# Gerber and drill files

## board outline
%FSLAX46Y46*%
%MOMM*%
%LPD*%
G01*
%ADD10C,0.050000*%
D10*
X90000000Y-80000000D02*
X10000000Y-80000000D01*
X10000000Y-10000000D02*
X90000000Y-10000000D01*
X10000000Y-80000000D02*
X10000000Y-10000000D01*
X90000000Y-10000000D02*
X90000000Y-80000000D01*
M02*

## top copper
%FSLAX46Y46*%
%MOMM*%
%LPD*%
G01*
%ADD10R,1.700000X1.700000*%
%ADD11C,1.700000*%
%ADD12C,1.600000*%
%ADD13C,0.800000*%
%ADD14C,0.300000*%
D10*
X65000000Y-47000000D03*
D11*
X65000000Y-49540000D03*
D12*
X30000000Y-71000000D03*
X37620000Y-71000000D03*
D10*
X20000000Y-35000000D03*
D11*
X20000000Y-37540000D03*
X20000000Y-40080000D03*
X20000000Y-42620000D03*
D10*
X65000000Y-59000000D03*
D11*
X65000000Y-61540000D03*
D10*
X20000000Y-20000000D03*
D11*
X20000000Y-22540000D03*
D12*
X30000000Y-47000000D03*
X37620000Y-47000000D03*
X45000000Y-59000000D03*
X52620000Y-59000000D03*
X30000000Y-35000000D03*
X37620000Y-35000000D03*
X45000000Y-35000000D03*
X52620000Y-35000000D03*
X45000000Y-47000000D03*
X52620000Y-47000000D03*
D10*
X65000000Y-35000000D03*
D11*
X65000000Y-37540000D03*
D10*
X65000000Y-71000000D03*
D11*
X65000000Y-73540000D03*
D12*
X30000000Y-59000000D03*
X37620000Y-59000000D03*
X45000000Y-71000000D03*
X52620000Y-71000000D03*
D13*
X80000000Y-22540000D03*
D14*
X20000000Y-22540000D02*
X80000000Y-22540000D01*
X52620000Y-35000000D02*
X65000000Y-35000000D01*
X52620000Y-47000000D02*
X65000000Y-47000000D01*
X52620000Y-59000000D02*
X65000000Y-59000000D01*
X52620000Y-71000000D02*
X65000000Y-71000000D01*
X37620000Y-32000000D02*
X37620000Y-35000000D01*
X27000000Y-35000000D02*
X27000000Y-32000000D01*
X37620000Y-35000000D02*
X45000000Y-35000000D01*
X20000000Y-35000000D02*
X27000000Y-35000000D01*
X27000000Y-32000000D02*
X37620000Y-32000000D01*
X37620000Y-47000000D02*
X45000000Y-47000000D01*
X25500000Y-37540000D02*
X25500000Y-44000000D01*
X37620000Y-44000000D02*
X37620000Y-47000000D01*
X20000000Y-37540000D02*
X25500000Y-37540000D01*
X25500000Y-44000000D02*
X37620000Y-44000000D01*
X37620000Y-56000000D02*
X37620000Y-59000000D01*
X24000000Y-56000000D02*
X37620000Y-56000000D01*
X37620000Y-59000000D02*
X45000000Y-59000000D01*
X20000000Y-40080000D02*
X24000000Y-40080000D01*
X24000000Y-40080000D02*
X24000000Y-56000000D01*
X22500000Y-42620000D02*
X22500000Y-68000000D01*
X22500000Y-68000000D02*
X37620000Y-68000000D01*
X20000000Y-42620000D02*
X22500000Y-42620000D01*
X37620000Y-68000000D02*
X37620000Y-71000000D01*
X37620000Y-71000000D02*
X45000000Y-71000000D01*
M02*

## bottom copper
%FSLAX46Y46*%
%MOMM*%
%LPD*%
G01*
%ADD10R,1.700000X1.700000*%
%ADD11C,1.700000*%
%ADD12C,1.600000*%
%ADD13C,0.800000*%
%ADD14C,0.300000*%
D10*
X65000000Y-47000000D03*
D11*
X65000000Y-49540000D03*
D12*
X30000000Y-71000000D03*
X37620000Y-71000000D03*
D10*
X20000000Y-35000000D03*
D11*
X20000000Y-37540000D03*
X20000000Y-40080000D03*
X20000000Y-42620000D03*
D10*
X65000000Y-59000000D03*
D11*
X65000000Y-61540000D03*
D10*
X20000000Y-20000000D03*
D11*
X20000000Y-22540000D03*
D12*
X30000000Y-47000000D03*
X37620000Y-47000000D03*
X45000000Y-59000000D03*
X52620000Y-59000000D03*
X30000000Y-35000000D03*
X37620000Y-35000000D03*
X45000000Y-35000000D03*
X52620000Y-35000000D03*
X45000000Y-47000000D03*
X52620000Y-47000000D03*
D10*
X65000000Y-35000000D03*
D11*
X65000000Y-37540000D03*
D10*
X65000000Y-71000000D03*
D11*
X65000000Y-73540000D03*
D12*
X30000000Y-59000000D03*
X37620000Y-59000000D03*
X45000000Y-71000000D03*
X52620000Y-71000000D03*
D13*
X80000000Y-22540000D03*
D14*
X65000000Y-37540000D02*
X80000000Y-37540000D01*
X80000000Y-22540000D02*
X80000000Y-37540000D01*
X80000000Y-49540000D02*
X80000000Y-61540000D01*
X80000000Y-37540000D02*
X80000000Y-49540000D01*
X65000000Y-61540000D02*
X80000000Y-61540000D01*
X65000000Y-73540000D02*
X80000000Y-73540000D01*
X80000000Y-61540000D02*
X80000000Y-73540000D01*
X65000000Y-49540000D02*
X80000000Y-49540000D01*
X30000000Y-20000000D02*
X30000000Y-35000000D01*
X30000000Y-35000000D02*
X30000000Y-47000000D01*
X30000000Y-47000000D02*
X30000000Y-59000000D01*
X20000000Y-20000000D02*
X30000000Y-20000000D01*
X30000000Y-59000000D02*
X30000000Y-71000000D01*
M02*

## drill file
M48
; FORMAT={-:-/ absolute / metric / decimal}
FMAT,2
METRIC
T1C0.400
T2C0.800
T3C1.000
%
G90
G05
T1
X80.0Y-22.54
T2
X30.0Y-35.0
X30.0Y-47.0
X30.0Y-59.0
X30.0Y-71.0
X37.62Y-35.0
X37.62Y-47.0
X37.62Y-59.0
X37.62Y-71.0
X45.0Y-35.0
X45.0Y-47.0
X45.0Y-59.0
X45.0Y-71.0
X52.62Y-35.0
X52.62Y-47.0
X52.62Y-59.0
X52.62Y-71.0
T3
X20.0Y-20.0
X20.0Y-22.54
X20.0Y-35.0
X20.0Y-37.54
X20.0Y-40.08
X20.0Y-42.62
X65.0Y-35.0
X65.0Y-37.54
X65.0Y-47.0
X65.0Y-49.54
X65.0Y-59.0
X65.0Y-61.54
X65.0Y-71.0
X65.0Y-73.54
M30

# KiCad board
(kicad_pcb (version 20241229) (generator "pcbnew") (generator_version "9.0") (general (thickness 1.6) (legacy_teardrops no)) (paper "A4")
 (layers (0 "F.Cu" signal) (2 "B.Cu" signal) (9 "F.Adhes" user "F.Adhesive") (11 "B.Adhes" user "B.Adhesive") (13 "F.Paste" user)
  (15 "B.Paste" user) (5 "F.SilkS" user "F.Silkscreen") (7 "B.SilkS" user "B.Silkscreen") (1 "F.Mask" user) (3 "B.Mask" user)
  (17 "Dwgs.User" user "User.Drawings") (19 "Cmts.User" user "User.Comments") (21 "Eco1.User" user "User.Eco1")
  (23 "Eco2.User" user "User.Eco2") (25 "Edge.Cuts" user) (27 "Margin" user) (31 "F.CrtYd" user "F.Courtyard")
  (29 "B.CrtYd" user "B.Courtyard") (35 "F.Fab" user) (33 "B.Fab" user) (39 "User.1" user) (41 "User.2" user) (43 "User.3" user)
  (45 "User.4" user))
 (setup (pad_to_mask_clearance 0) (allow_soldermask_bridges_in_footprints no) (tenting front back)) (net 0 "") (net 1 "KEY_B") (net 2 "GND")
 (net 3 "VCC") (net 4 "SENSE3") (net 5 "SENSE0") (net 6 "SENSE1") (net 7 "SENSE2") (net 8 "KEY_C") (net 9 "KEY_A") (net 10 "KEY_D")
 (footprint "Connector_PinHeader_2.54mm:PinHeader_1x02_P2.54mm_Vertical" (layer "F.Cu") (at 65 47)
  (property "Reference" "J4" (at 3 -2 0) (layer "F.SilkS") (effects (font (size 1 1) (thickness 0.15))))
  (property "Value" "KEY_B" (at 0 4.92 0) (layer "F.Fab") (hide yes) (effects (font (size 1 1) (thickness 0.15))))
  (pad "1" thru_hole rect (at 0 0) (size 1.7 1.7) (drill 1) (layers "*.Cu" "*.Mask") (remove_unused_layers no) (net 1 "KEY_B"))
  (pad "2" thru_hole circle (at 0 2.54) (size 1.7 1.7) (drill 1) (layers "*.Cu" "*.Mask") (remove_unused_layers no) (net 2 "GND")))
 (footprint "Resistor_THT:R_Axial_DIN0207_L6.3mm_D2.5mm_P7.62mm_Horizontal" (layer "F.Cu") (at 30 71)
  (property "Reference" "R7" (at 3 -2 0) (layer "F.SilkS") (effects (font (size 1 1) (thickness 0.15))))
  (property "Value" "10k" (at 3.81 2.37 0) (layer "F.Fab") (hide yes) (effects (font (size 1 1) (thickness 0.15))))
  (pad "1" thru_hole circle (at 0 0) (size 1.6 1.6) (drill 0.8) (layers "*.Cu" "*.Mask") (remove_unused_layers no) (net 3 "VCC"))
  (pad "2" thru_hole circle (at 7.62 0) (size 1.6 1.6) (drill 0.8) (layers "*.Cu" "*.Mask") (remove_unused_layers no) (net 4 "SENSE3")))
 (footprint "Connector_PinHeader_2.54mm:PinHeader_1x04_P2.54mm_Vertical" (layer "F.Cu") (at 20 35)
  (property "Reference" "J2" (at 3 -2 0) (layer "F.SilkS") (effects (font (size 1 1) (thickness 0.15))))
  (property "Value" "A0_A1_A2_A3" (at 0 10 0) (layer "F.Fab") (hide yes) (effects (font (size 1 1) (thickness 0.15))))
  (pad "1" thru_hole rect (at 0 0) (size 1.7 1.7) (drill 1) (layers "*.Cu" "*.Mask") (remove_unused_layers no) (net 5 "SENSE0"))
  (pad "2" thru_hole circle (at 0 2.54) (size 1.7 1.7) (drill 1) (layers "*.Cu" "*.Mask") (remove_unused_layers no) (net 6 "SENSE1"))
  (pad "3" thru_hole circle (at 0 5.08) (size 1.7 1.7) (drill 1) (layers "*.Cu" "*.Mask") (remove_unused_layers no) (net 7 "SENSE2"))
  (pad "4" thru_hole circle (at 0 7.62) (size 1.7 1.7) (drill 1) (layers "*.Cu" "*.Mask") (remove_unused_layers no) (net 4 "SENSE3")))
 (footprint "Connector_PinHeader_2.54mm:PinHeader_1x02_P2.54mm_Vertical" (layer "F.Cu") (at 65 59)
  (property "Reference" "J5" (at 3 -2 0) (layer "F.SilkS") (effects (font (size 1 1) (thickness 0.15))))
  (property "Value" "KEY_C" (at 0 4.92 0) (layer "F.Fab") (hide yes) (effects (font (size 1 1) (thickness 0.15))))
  (pad "1" thru_hole rect (at 0 0) (size 1.7 1.7) (drill 1) (layers "*.Cu" "*.Mask") (remove_unused_layers no) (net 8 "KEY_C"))
  (pad "2" thru_hole circle (at 0 2.54) (size 1.7 1.7) (drill 1) (layers "*.Cu" "*.Mask") (remove_unused_layers no) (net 2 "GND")))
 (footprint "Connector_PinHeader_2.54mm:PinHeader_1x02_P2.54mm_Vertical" (layer "F.Cu") (at 20 20)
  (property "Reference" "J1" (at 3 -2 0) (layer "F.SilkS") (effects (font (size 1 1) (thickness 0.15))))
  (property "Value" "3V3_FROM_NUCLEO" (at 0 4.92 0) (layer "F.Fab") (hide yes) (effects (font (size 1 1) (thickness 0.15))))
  (pad "1" thru_hole rect (at 0 0) (size 1.7 1.7) (drill 1) (layers "*.Cu" "*.Mask") (remove_unused_layers no) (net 3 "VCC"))
  (pad "2" thru_hole circle (at 0 2.54) (size 1.7 1.7) (drill 1) (layers "*.Cu" "*.Mask") (remove_unused_layers no) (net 2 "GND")))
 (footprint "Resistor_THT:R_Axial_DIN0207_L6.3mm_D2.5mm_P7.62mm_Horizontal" (layer "F.Cu") (at 30 47)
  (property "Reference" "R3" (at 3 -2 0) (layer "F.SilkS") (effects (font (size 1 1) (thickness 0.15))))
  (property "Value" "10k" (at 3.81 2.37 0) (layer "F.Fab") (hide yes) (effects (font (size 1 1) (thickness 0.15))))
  (pad "1" thru_hole circle (at 0 0) (size 1.6 1.6) (drill 0.8) (layers "*.Cu" "*.Mask") (remove_unused_layers no) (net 3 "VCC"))
  (pad "2" thru_hole circle (at 7.62 0) (size 1.6 1.6) (drill 0.8) (layers "*.Cu" "*.Mask") (remove_unused_layers no) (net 6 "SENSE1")))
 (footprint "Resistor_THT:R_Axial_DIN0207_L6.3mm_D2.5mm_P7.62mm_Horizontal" (layer "F.Cu") (at 45 59)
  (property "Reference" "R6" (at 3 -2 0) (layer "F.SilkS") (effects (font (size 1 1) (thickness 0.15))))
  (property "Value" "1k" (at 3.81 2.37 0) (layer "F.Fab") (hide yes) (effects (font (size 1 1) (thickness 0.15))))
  (pad "1" thru_hole circle (at 0 0) (size 1.6 1.6) (drill 0.8) (layers "*.Cu" "*.Mask") (remove_unused_layers no) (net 7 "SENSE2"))
  (pad "2" thru_hole circle (at 7.62 0) (size 1.6 1.6) (drill 0.8) (layers "*.Cu" "*.Mask") (remove_unused_layers no) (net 8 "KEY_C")))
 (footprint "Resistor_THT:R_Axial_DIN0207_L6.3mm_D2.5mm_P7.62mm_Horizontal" (layer "F.Cu") (at 30 35)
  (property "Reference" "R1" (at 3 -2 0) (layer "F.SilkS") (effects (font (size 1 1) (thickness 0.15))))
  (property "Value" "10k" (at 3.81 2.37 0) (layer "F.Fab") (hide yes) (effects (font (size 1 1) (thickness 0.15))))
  (pad "1" thru_hole circle (at 0 0) (size 1.6 1.6) (drill 0.8) (layers "*.Cu" "*.Mask") (remove_unused_layers no) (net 3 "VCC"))
  (pad "2" thru_hole circle (at 7.62 0) (size 1.6 1.6) (drill 0.8) (layers "*.Cu" "*.Mask") (remove_unused_layers no) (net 5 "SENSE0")))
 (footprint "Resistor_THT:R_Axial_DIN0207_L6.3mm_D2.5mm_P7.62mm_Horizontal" (layer "F.Cu") (at 45 35)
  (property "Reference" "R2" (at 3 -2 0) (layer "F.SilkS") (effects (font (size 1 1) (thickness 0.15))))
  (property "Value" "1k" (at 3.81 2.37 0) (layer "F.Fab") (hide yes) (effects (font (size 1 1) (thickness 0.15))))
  (pad "1" thru_hole circle (at 0 0) (size 1.6 1.6) (drill 0.8) (layers "*.Cu" "*.Mask") (remove_unused_layers no) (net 5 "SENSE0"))
  (pad "2" thru_hole circle (at 7.62 0) (size 1.6 1.6) (drill 0.8) (layers "*.Cu" "*.Mask") (remove_unused_layers no) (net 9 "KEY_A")))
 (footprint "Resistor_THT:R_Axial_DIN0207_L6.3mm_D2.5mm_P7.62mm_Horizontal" (layer "F.Cu") (at 45 47)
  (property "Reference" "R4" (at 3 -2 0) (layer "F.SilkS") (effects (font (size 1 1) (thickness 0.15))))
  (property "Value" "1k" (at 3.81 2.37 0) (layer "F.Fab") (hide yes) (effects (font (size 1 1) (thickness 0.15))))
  (pad "1" thru_hole circle (at 0 0) (size 1.6 1.6) (drill 0.8) (layers "*.Cu" "*.Mask") (remove_unused_layers no) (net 6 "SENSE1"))
  (pad "2" thru_hole circle (at 7.62 0) (size 1.6 1.6) (drill 0.8) (layers "*.Cu" "*.Mask") (remove_unused_layers no) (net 1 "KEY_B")))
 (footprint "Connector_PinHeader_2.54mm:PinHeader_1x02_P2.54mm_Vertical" (layer "F.Cu") (at 65 35)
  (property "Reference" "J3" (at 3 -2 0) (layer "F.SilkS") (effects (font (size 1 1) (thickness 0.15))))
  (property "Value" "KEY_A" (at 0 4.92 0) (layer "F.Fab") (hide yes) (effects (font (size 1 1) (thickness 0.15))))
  (pad "1" thru_hole rect (at 0 0) (size 1.7 1.7) (drill 1) (layers "*.Cu" "*.Mask") (remove_unused_layers no) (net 9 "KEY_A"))
  (pad "2" thru_hole circle (at 0 2.54) (size 1.7 1.7) (drill 1) (layers "*.Cu" "*.Mask") (remove_unused_layers no) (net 2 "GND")))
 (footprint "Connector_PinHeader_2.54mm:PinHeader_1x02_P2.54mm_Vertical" (layer "F.Cu") (at 65 71)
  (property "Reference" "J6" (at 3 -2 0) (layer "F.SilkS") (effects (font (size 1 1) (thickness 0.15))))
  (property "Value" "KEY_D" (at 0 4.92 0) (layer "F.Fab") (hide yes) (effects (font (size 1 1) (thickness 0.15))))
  (pad "1" thru_hole rect (at 0 0) (size 1.7 1.7) (drill 1) (layers "*.Cu" "*.Mask") (remove_unused_layers no) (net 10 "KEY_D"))
  (pad "2" thru_hole circle (at 0 2.54) (size 1.7 1.7) (drill 1) (layers "*.Cu" "*.Mask") (remove_unused_layers no) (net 2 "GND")))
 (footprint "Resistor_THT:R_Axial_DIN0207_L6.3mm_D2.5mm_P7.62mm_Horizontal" (layer "F.Cu") (at 30 59)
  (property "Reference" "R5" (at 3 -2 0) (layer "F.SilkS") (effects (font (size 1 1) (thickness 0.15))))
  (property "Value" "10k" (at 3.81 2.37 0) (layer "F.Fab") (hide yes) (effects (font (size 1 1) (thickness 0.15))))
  (pad "1" thru_hole circle (at 0 0) (size 1.6 1.6) (drill 0.8) (layers "*.Cu" "*.Mask") (remove_unused_layers no) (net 3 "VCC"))
  (pad "2" thru_hole circle (at 7.62 0) (size 1.6 1.6) (drill 0.8) (layers "*.Cu" "*.Mask") (remove_unused_layers no) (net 7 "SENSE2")))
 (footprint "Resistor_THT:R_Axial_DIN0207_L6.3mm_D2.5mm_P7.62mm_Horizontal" (layer "F.Cu") (at 45 71)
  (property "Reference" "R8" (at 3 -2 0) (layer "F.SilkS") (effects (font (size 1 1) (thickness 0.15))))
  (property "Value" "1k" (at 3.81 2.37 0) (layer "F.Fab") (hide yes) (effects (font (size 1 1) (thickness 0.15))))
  (pad "1" thru_hole circle (at 0 0) (size 1.6 1.6) (drill 0.8) (layers "*.Cu" "*.Mask") (remove_unused_layers no) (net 4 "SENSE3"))
  (pad "2" thru_hole circle (at 7.62 0) (size 1.6 1.6) (drill 0.8) (layers "*.Cu" "*.Mask") (remove_unused_layers no) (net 10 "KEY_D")))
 (gr_line (start 90 80) (end 10 80) (stroke (width 0.05) (type default)) (layer "Edge.Cuts"))
 (gr_line (start 10 10) (end 90 10) (stroke (width 0.05) (type default)) (layer "Edge.Cuts"))
 (gr_line (start 10 80) (end 10 10) (stroke (width 0.05) (type default)) (layer "Edge.Cuts"))
 (gr_line (start 90 10) (end 90 80) (stroke (width 0.05) (type default)) (layer "Edge.Cuts"))
 (segment (start 20 22.54) (end 80 22.54) (width 0.3) (layer "F.Cu") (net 2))
 (via (at 80 22.54) (size 0.8) (drill 0.4) (layers "F.Cu" "B.Cu") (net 2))
 (segment (start 65 37.54) (end 80 37.54) (width 0.3) (layer "B.Cu") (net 2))
 (segment (start 80 22.54) (end 80 37.54) (width 0.3) (layer "B.Cu") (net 2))
 (segment (start 80 49.54) (end 80 61.54) (width 0.3) (layer "B.Cu") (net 2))
 (segment (start 80 37.54) (end 80 49.54) (width 0.3) (layer "B.Cu") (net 2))
 (segment (start 65 61.54) (end 80 61.54) (width 0.3) (layer "B.Cu") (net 2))
 (segment (start 65 73.54) (end 80 73.54) (width 0.3) (layer "B.Cu") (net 2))
 (segment (start 80 61.54) (end 80 73.54) (width 0.3) (layer "B.Cu") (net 2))
 (segment (start 65 49.54) (end 80 49.54) (width 0.3) (layer "B.Cu") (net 2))
 (segment (start 52.62 35) (end 65 35) (width 0.3) (layer "F.Cu") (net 9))
 (segment (start 52.62 47) (end 65 47) (width 0.3) (layer "F.Cu") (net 1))
 (segment (start 52.62 59) (end 65 59) (width 0.3) (layer "F.Cu") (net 8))
 (segment (start 52.62 71) (end 65 71) (width 0.3) (layer "F.Cu") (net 10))
 (segment (start 37.62 32) (end 37.62 35) (width 0.3) (layer "F.Cu") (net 5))
 (segment (start 27 35) (end 27 32) (width 0.3) (layer "F.Cu") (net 5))
 (segment (start 37.62 35) (end 45 35) (width 0.3) (layer "F.Cu") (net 5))
 (segment (start 20 35) (end 27 35) (width 0.3) (layer "F.Cu") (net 5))
 (segment (start 27 32) (end 37.62 32) (width 0.3) (layer "F.Cu") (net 5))
 (segment (start 37.62 47) (end 45 47) (width 0.3) (layer "F.Cu") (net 6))
 (segment (start 25.5 37.54) (end 25.5 44) (width 0.3) (layer "F.Cu") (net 6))
 (segment (start 37.62 44) (end 37.62 47) (width 0.3) (layer "F.Cu") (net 6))
 (segment (start 20 37.54) (end 25.5 37.54) (width 0.3) (layer "F.Cu") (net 6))
 (segment (start 25.5 44) (end 37.62 44) (width 0.3) (layer "F.Cu") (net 6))
 (segment (start 37.62 56) (end 37.62 59) (width 0.3) (layer "F.Cu") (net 7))
 (segment (start 24 56) (end 37.62 56) (width 0.3) (layer "F.Cu") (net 7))
 (segment (start 37.62 59) (end 45 59) (width 0.3) (layer "F.Cu") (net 7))
 (segment (start 20 40.08) (end 24 40.08) (width 0.3) (layer "F.Cu") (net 7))
 (segment (start 24 40.08) (end 24 56) (width 0.3) (layer "F.Cu") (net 7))
 (segment (start 22.5 42.62) (end 22.5 68) (width 0.3) (layer "F.Cu") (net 4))
 (segment (start 22.5 68) (end 37.62 68) (width 0.3) (layer "F.Cu") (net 4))
 (segment (start 20 42.62) (end 22.5 42.62) (width 0.3) (layer "F.Cu") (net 4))
 (segment (start 37.62 68) (end 37.62 71) (width 0.3) (layer "F.Cu") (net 4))
 (segment (start 37.62 71) (end 45 71) (width 0.3) (layer "F.Cu") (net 4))
 (segment (start 30 20) (end 30 35) (width 0.3) (layer "B.Cu") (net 3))
 (segment (start 30 35) (end 30 47) (width 0.3) (layer "B.Cu") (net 3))
 (segment (start 30 47) (end 30 59) (width 0.3) (layer "B.Cu") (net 3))
 (segment (start 20 20) (end 30 20) (width 0.3) (layer "B.Cu") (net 3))
 (segment (start 30 59) (end 30 71) (width 0.3) (layer "B.Cu") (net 3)))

